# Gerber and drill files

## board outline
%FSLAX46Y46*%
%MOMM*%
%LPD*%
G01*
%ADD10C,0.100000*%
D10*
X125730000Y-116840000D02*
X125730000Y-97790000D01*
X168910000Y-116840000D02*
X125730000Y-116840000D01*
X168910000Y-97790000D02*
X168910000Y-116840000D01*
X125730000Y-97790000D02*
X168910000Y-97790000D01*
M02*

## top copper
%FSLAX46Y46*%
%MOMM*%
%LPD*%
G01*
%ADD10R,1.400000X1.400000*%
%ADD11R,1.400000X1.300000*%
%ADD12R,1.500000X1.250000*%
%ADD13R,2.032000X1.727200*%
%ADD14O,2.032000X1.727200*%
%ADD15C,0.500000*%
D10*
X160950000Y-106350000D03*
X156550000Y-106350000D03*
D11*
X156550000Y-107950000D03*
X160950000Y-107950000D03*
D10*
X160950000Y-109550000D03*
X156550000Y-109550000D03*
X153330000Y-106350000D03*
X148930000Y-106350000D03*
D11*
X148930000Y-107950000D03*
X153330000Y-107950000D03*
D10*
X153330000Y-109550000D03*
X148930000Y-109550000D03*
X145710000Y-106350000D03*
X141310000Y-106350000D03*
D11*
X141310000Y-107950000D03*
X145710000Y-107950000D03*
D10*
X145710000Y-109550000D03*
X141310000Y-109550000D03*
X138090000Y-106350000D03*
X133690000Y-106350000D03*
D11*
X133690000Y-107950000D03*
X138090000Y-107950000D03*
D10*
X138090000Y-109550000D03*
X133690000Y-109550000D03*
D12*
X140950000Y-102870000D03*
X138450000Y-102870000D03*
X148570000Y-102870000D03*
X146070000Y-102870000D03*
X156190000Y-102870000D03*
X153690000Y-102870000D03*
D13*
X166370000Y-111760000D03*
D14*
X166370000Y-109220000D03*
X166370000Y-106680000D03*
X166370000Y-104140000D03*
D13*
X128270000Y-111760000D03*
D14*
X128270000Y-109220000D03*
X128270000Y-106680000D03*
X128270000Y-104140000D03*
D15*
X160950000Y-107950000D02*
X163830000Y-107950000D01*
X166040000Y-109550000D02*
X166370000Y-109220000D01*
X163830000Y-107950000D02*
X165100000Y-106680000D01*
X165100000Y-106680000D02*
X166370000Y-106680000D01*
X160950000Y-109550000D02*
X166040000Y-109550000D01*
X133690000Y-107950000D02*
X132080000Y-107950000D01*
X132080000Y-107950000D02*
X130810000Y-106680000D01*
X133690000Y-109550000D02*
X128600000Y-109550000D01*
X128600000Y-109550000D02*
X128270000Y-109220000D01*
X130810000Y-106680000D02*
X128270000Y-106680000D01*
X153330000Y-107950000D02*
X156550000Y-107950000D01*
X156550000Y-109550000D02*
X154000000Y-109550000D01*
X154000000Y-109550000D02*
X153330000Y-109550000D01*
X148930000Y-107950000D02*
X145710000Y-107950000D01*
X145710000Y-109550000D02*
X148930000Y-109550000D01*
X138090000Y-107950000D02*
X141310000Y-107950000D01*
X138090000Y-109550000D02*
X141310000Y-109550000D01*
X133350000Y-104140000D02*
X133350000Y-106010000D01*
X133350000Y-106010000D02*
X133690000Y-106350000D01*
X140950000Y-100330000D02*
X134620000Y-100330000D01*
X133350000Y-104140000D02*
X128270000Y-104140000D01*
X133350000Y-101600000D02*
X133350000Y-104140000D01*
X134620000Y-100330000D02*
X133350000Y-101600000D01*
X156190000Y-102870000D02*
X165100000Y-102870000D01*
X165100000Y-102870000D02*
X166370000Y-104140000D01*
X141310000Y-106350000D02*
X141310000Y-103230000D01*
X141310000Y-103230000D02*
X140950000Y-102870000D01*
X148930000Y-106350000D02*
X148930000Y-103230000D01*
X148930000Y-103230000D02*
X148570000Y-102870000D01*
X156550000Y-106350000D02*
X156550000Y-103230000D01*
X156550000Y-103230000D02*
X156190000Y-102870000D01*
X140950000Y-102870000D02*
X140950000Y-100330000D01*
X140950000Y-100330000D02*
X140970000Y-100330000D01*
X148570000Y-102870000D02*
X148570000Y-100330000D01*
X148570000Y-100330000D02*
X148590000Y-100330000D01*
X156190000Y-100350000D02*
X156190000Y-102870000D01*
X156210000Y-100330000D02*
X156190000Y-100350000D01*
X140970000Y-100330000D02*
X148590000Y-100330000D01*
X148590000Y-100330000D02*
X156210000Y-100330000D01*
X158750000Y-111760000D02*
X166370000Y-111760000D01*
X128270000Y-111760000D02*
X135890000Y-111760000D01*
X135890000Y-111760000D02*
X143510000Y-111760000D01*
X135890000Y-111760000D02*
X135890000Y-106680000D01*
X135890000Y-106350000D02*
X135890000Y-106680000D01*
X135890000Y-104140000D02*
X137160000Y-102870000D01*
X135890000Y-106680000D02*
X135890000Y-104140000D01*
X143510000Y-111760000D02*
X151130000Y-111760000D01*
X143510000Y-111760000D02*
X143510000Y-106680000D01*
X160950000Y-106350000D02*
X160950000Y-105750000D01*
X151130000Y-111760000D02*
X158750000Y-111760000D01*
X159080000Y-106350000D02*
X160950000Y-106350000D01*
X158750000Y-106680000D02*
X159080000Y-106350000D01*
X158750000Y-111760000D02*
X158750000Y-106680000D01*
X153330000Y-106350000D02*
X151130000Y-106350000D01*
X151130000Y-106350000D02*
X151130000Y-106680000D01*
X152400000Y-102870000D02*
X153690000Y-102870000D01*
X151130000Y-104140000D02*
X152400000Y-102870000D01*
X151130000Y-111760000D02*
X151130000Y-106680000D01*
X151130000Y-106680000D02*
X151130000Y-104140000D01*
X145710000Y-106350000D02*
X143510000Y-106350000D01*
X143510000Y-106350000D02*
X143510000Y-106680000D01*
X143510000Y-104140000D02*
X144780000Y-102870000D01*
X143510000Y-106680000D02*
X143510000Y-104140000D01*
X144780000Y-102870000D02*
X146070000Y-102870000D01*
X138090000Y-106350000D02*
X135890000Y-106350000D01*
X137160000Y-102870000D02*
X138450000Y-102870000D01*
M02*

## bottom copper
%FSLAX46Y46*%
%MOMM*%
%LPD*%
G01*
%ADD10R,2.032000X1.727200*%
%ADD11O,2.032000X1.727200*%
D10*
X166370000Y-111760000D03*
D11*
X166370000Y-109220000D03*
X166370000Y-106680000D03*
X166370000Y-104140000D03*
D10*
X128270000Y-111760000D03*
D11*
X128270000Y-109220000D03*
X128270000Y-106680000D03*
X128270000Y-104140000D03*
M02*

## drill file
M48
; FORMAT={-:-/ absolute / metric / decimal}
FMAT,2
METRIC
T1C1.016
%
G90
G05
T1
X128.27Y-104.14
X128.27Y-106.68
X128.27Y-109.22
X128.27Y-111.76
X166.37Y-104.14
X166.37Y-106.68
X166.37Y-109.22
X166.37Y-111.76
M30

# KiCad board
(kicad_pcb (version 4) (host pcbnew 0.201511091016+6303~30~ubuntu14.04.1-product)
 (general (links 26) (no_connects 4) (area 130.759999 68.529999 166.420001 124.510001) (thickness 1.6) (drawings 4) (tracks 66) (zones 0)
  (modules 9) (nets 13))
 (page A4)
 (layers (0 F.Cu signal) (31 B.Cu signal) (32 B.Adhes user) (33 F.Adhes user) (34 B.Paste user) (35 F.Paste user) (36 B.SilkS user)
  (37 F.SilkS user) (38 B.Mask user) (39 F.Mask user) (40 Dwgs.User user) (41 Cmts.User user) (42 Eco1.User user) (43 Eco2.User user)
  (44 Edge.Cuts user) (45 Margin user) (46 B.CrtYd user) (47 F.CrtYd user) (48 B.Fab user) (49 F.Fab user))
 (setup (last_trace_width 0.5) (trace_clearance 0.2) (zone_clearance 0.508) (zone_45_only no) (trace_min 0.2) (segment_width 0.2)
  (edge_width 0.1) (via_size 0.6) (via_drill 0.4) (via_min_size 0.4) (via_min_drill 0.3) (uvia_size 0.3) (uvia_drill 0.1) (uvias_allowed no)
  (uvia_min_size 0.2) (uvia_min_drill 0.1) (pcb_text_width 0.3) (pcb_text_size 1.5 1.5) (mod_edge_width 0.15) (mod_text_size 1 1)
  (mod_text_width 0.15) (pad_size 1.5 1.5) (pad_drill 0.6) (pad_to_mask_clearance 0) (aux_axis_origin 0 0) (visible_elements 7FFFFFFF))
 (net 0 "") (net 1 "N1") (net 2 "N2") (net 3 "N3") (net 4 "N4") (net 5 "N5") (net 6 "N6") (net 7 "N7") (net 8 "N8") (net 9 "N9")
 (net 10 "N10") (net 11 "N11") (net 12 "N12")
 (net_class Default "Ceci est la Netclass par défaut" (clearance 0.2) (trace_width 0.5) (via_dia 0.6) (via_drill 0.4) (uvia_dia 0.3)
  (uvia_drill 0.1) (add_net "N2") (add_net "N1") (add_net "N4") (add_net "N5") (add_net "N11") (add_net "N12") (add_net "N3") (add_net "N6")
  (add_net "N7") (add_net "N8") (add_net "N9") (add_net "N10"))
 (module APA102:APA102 (layer F.Cu) (at 158.75 107.95 90)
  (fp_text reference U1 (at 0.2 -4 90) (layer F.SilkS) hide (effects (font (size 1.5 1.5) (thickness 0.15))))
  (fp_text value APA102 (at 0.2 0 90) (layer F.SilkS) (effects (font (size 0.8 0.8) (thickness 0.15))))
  (pad 3 smd rect (at 1.6 2.2 180) (size 1.4 1.4) (layers F.Cu F.Paste F.Mask) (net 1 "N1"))
  (pad 4 smd rect (at 1.6 -2.2 180) (size 1.4 1.4) (layers F.Cu F.Paste F.Mask) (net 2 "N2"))
  (pad 5 smd rect (at 0 -2.2 180) (size 1.4 1.3) (layers F.Cu F.Paste F.Mask) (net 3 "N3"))
  (pad 2 smd rect (at 0 2.2 180) (size 1.4 1.3) (layers F.Cu F.Paste F.Mask) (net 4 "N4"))
  (pad 1 smd rect (at -1.6 2.2 180) (size 1.4 1.4) (layers F.Cu F.Paste F.Mask) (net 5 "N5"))
  (pad 6 smd rect (at -1.6 -2.2 180) (size 1.4 1.4) (layers F.Cu F.Paste F.Mask) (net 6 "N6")))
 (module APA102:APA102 (layer F.Cu) (at 151.13 107.95 90)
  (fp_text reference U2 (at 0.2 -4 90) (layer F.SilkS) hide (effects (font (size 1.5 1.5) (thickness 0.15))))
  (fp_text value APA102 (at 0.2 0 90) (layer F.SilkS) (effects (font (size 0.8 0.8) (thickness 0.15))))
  (pad 3 smd rect (at 1.6 2.2 180) (size 1.4 1.4) (layers F.Cu F.Paste F.Mask) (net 1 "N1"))
  (pad 4 smd rect (at 1.6 -2.2 180) (size 1.4 1.4) (layers F.Cu F.Paste F.Mask) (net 2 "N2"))
  (pad 5 smd rect (at 0 -2.2 180) (size 1.4 1.3) (layers F.Cu F.Paste F.Mask) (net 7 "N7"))
  (pad 2 smd rect (at 0 2.2 180) (size 1.4 1.3) (layers F.Cu F.Paste F.Mask) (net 3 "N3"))
  (pad 1 smd rect (at -1.6 2.2 180) (size 1.4 1.4) (layers F.Cu F.Paste F.Mask) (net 6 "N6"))
  (pad 6 smd rect (at -1.6 -2.2 180) (size 1.4 1.4) (layers F.Cu F.Paste F.Mask) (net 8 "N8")))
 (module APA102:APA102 (layer F.Cu) (at 143.51 107.95 90)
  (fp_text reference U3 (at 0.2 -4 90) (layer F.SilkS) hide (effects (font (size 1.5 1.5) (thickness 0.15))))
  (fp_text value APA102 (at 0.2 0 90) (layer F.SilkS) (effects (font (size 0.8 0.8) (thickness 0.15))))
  (pad 3 smd rect (at 1.6 2.2 180) (size 1.4 1.4) (layers F.Cu F.Paste F.Mask) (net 1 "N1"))
  (pad 4 smd rect (at 1.6 -2.2 180) (size 1.4 1.4) (layers F.Cu F.Paste F.Mask) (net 2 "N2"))
  (pad 5 smd rect (at 0 -2.2 180) (size 1.4 1.3) (layers F.Cu F.Paste F.Mask) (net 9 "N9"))
  (pad 2 smd rect (at 0 2.2 180) (size 1.4 1.3) (layers F.Cu F.Paste F.Mask) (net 7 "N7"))
  (pad 1 smd rect (at -1.6 2.2 180) (size 1.4 1.4) (layers F.Cu F.Paste F.Mask) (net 8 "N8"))
  (pad 6 smd rect (at -1.6 -2.2 180) (size 1.4 1.4) (layers F.Cu F.Paste F.Mask) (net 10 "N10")))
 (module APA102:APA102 (layer F.Cu) (at 135.89 107.95 90)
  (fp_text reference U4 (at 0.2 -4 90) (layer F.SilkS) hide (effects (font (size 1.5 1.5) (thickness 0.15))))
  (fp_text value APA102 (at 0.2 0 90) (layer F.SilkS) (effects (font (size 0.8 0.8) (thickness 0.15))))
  (pad 3 smd rect (at 1.6 2.2 180) (size 1.4 1.4) (layers F.Cu F.Paste F.Mask) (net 1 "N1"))
  (pad 4 smd rect (at 1.6 -2.2 180) (size 1.4 1.4) (layers F.Cu F.Paste F.Mask) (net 2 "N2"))
  (pad 5 smd rect (at 0 -2.2 180) (size 1.4 1.3) (layers F.Cu F.Paste F.Mask) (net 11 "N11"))
  (pad 2 smd rect (at 0 2.2 180) (size 1.4 1.3) (layers F.Cu F.Paste F.Mask) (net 9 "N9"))
  (pad 1 smd rect (at -1.6 2.2 180) (size 1.4 1.4) (layers F.Cu F.Paste F.Mask) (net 10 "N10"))
  (pad 6 smd rect (at -1.6 -2.2 180) (size 1.4 1.4) (layers F.Cu F.Paste F.Mask) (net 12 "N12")))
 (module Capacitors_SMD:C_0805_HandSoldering (layer F.Cu) (at 139.7 102.87 180)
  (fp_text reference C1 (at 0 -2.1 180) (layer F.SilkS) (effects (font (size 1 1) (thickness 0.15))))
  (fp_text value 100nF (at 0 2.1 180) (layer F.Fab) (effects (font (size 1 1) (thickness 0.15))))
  (pad 1 smd rect (at -1.25 0 180) (size 1.5 1.25) (layers F.Cu F.Paste F.Mask) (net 2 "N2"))
  (pad 2 smd rect (at 1.25 0 180) (size 1.5 1.25) (layers F.Cu F.Paste F.Mask) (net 1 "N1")))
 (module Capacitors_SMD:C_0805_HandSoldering (layer F.Cu) (at 147.32 102.87 180)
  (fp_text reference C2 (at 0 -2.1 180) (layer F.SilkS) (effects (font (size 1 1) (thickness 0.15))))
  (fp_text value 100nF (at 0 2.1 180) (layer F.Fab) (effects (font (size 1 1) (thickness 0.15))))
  (pad 1 smd rect (at -1.25 0 180) (size 1.5 1.25) (layers F.Cu F.Paste F.Mask) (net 2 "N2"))
  (pad 2 smd rect (at 1.25 0 180) (size 1.5 1.25) (layers F.Cu F.Paste F.Mask) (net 1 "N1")))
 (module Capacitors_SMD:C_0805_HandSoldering (layer F.Cu) (at 154.94 102.87 180)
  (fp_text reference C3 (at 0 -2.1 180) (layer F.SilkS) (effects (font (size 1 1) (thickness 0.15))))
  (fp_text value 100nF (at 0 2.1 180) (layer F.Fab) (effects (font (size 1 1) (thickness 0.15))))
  (pad 1 smd rect (at -1.25 0 180) (size 1.5 1.25) (layers F.Cu F.Paste F.Mask) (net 2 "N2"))
  (pad 2 smd rect (at 1.25 0 180) (size 1.5 1.25) (layers F.Cu F.Paste F.Mask) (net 1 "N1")))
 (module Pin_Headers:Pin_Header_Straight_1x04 (layer F.Cu) (at 166.37 111.76 180)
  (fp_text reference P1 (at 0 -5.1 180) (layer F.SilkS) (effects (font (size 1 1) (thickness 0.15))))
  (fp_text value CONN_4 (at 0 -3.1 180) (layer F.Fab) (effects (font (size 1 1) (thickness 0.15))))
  (pad 1 thru_hole rect (at 0 0 180) (size 2.032 1.7272) (drill 1.016) (layers *.Cu *.Mask F.SilkS) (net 1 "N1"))
  (pad 2 thru_hole oval (at 0 2.54 180) (size 2.032 1.7272) (drill 1.016) (layers *.Cu *.Mask F.SilkS) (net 4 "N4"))
  (pad 3 thru_hole oval (at 0 5.08 180) (size 2.032 1.7272) (drill 1.016) (layers *.Cu *.Mask F.SilkS) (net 5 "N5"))
  (pad 4 thru_hole oval (at 0 7.62 180) (size 2.032 1.7272) (drill 1.016) (layers *.Cu *.Mask F.SilkS) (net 2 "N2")))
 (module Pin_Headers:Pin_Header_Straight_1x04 (layer F.Cu) (at 128.27 111.76 180)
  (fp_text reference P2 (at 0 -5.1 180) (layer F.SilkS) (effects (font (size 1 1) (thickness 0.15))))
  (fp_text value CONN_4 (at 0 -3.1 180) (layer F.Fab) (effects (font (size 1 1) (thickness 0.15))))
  (pad 1 thru_hole rect (at 0 0 180) (size 2.032 1.7272) (drill 1.016) (layers *.Cu *.Mask F.SilkS) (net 1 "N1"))
  (pad 2 thru_hole oval (at 0 2.54 180) (size 2.032 1.7272) (drill 1.016) (layers *.Cu *.Mask F.SilkS) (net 11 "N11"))
  (pad 3 thru_hole oval (at 0 5.08 180) (size 2.032 1.7272) (drill 1.016) (layers *.Cu *.Mask F.SilkS) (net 12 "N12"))
  (pad 4 thru_hole oval (at 0 7.62 180) (size 2.032 1.7272) (drill 1.016) (layers *.Cu *.Mask F.SilkS) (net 2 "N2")))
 (gr_line (start 125.73 116.84) (end 125.73 97.79) (angle 90) (layer Edge.Cuts) (width 0.1))
 (gr_line (start 168.91 116.84) (end 125.73 116.84) (angle 90) (layer Edge.Cuts) (width 0.1))
 (gr_line (start 168.91 97.79) (end 168.91 116.84) (angle 90) (layer Edge.Cuts) (width 0.1))
 (gr_line (start 125.73 97.79) (end 168.91 97.79) (angle 90) (layer Edge.Cuts) (width 0.1))
 (segment (start 160.95 107.95) (end 163.83 107.95) (width 0.5) (layer F.Cu) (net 4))
 (segment (start 166.04 109.55) (end 166.37 109.22) (width 0.5) (layer F.Cu) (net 4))
 (segment (start 163.83 107.95) (end 165.1 106.68) (width 0.5) (layer F.Cu) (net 4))
 (segment (start 165.1 106.68) (end 166.37 106.68) (width 0.5) (layer F.Cu) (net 5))
 (segment (start 160.95 109.55) (end 166.04 109.55) (width 0.5) (layer F.Cu) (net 5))
 (segment (start 133.69 107.95) (end 132.08 107.95) (width 0.5) (layer F.Cu) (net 11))
 (segment (start 132.08 107.95) (end 130.81 106.68) (width 0.5) (layer F.Cu) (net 11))
 (segment (start 133.69 109.55) (end 128.6 109.55) (width 0.5) (layer F.Cu) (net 11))
 (segment (start 128.6 109.55) (end 128.27 109.22) (width 0.5) (layer F.Cu) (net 11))
 (segment (start 130.81 106.68) (end 128.27 106.68) (width 0.5) (layer F.Cu) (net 12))
 (segment (start 153.33 107.95) (end 156.55 107.95) (width 0.5) (layer F.Cu) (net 3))
 (segment (start 156.55 109.55) (end 154 109.55) (width 0.5) (layer F.Cu) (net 6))
 (segment (start 154 109.55) (end 153.33 109.55) (width 0.5) (layer F.Cu) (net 6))
 (segment (start 148.93 107.95) (end 145.71 107.95) (width 0.5) (layer F.Cu) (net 7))
 (segment (start 145.71 109.55) (end 148.93 109.55) (width 0.5) (layer F.Cu) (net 8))
 (segment (start 138.09 107.95) (end 141.31 107.95) (width 0.5) (layer F.Cu) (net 9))
 (segment (start 138.09 109.55) (end 141.31 109.55) (width 0.5) (layer F.Cu) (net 10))
 (segment (start 133.35 104.14) (end 133.35 106.01) (width 0.5) (layer F.Cu) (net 2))
 (segment (start 133.35 106.01) (end 133.69 106.35) (width 0.5) (layer F.Cu) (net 2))
 (segment (start 140.95 100.33) (end 134.62 100.33) (width 0.5) (layer F.Cu) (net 2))
 (segment (start 133.35 104.14) (end 128.27 104.14) (width 0.5) (layer F.Cu) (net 2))
 (segment (start 133.35 101.6) (end 133.35 104.14) (width 0.5) (layer F.Cu) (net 2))
 (segment (start 134.62 100.33) (end 133.35 101.6) (width 0.5) (layer F.Cu) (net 2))
 (segment (start 156.19 102.87) (end 165.1 102.87) (width 0.5) (layer F.Cu) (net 2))
 (segment (start 165.1 102.87) (end 166.37 104.14) (width 0.5) (layer F.Cu) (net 2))
 (segment (start 141.31 106.35) (end 141.31 103.23) (width 0.5) (layer F.Cu) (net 2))
 (segment (start 141.31 103.23) (end 140.95 102.87) (width 0.5) (layer F.Cu) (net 2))
 (segment (start 148.93 106.35) (end 148.93 103.23) (width 0.5) (layer F.Cu) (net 2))
 (segment (start 148.93 103.23) (end 148.57 102.87) (width 0.5) (layer F.Cu) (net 2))
 (segment (start 156.55 106.35) (end 156.55 103.23) (width 0.5) (layer F.Cu) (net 2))
 (segment (start 156.55 103.23) (end 156.19 102.87) (width 0.5) (layer F.Cu) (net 2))
 (segment (start 140.95 102.87) (end 140.95 100.33) (width 0.5) (layer F.Cu) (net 2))
 (segment (start 140.95 100.33) (end 140.97 100.33) (width 0.5) (layer F.Cu) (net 2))
 (segment (start 148.57 102.87) (end 148.57 100.33) (width 0.5) (layer F.Cu) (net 2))
 (segment (start 148.57 100.33) (end 148.59 100.33) (width 0.5) (layer F.Cu) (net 2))
 (segment (start 156.19 100.35) (end 156.19 102.87) (width 0.5) (layer F.Cu) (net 2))
 (segment (start 156.21 100.33) (end 156.19 100.35) (width 0.5) (layer F.Cu) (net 2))
 (segment (start 140.97 100.33) (end 148.59 100.33) (width 0.5) (layer F.Cu) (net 2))
 (segment (start 148.59 100.33) (end 156.21 100.33) (width 0.5) (layer F.Cu) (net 2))
 (segment (start 158.75 111.76) (end 166.37 111.76) (width 0.5) (layer F.Cu) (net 1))
 (segment (start 128.27 111.76) (end 135.89 111.76) (width 0.5) (layer F.Cu) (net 1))
 (segment (start 135.89 111.76) (end 143.51 111.76) (width 0.5) (layer F.Cu) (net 1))
 (segment (start 135.89 111.76) (end 135.89 106.68) (width 0.5) (layer F.Cu) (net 1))
 (segment (start 135.89 106.35) (end 135.89 106.68) (width 0.5) (layer F.Cu) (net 1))
 (segment (start 135.89 104.14) (end 137.16 102.87) (width 0.5) (layer F.Cu) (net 1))
 (segment (start 135.89 106.68) (end 135.89 104.14) (width 0.5) (layer F.Cu) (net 1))
 (segment (start 143.51 111.76) (end 151.13 111.76) (width 0.5) (layer F.Cu) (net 1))
 (segment (start 143.51 111.76) (end 143.51 106.68) (width 0.5) (layer F.Cu) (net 1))
 (segment (start 160.95 106.35) (end 160.95 105.75) (width 0.5) (layer F.Cu) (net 1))
 (segment (start 151.13 111.76) (end 158.75 111.76) (width 0.5) (layer F.Cu) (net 1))
 (segment (start 159.08 106.35) (end 160.95 106.35) (width 0.5) (layer F.Cu) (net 1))
 (segment (start 158.75 106.68) (end 159.08 106.35) (width 0.5) (layer F.Cu) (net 1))
 (segment (start 158.75 111.76) (end 158.75 106.68) (width 0.5) (layer F.Cu) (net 1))
 (segment (start 153.33 106.35) (end 151.13 106.35) (width 0.5) (layer F.Cu) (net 1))
 (segment (start 151.13 106.35) (end 151.13 106.68) (width 0.5) (layer F.Cu) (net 1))
 (segment (start 152.4 102.87) (end 153.69 102.87) (width 0.5) (layer F.Cu) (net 1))
 (segment (start 151.13 104.14) (end 152.4 102.87) (width 0.5) (layer F.Cu) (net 1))
 (segment (start 151.13 111.76) (end 151.13 106.68) (width 0.5) (layer F.Cu) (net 1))
 (segment (start 151.13 106.68) (end 151.13 104.14) (width 0.5) (layer F.Cu) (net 1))
 (segment (start 145.71 106.35) (end 143.51 106.35) (width 0.5) (layer F.Cu) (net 1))
 (segment (start 143.51 106.35) (end 143.51 106.68) (width 0.5) (layer F.Cu) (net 1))
 (segment (start 143.51 104.14) (end 144.78 102.87) (width 0.5) (layer F.Cu) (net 1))
 (segment (start 143.51 106.68) (end 143.51 104.14) (width 0.5) (layer F.Cu) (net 1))
 (segment (start 144.78 102.87) (end 146.07 102.87) (width 0.5) (layer F.Cu) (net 1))
 (segment (start 138.09 106.35) (end 135.89 106.35) (width 0.5) (layer F.Cu) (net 1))
 (segment (start 137.16 102.87) (end 138.45 102.87) (width 0.5) (layer F.Cu) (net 1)))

